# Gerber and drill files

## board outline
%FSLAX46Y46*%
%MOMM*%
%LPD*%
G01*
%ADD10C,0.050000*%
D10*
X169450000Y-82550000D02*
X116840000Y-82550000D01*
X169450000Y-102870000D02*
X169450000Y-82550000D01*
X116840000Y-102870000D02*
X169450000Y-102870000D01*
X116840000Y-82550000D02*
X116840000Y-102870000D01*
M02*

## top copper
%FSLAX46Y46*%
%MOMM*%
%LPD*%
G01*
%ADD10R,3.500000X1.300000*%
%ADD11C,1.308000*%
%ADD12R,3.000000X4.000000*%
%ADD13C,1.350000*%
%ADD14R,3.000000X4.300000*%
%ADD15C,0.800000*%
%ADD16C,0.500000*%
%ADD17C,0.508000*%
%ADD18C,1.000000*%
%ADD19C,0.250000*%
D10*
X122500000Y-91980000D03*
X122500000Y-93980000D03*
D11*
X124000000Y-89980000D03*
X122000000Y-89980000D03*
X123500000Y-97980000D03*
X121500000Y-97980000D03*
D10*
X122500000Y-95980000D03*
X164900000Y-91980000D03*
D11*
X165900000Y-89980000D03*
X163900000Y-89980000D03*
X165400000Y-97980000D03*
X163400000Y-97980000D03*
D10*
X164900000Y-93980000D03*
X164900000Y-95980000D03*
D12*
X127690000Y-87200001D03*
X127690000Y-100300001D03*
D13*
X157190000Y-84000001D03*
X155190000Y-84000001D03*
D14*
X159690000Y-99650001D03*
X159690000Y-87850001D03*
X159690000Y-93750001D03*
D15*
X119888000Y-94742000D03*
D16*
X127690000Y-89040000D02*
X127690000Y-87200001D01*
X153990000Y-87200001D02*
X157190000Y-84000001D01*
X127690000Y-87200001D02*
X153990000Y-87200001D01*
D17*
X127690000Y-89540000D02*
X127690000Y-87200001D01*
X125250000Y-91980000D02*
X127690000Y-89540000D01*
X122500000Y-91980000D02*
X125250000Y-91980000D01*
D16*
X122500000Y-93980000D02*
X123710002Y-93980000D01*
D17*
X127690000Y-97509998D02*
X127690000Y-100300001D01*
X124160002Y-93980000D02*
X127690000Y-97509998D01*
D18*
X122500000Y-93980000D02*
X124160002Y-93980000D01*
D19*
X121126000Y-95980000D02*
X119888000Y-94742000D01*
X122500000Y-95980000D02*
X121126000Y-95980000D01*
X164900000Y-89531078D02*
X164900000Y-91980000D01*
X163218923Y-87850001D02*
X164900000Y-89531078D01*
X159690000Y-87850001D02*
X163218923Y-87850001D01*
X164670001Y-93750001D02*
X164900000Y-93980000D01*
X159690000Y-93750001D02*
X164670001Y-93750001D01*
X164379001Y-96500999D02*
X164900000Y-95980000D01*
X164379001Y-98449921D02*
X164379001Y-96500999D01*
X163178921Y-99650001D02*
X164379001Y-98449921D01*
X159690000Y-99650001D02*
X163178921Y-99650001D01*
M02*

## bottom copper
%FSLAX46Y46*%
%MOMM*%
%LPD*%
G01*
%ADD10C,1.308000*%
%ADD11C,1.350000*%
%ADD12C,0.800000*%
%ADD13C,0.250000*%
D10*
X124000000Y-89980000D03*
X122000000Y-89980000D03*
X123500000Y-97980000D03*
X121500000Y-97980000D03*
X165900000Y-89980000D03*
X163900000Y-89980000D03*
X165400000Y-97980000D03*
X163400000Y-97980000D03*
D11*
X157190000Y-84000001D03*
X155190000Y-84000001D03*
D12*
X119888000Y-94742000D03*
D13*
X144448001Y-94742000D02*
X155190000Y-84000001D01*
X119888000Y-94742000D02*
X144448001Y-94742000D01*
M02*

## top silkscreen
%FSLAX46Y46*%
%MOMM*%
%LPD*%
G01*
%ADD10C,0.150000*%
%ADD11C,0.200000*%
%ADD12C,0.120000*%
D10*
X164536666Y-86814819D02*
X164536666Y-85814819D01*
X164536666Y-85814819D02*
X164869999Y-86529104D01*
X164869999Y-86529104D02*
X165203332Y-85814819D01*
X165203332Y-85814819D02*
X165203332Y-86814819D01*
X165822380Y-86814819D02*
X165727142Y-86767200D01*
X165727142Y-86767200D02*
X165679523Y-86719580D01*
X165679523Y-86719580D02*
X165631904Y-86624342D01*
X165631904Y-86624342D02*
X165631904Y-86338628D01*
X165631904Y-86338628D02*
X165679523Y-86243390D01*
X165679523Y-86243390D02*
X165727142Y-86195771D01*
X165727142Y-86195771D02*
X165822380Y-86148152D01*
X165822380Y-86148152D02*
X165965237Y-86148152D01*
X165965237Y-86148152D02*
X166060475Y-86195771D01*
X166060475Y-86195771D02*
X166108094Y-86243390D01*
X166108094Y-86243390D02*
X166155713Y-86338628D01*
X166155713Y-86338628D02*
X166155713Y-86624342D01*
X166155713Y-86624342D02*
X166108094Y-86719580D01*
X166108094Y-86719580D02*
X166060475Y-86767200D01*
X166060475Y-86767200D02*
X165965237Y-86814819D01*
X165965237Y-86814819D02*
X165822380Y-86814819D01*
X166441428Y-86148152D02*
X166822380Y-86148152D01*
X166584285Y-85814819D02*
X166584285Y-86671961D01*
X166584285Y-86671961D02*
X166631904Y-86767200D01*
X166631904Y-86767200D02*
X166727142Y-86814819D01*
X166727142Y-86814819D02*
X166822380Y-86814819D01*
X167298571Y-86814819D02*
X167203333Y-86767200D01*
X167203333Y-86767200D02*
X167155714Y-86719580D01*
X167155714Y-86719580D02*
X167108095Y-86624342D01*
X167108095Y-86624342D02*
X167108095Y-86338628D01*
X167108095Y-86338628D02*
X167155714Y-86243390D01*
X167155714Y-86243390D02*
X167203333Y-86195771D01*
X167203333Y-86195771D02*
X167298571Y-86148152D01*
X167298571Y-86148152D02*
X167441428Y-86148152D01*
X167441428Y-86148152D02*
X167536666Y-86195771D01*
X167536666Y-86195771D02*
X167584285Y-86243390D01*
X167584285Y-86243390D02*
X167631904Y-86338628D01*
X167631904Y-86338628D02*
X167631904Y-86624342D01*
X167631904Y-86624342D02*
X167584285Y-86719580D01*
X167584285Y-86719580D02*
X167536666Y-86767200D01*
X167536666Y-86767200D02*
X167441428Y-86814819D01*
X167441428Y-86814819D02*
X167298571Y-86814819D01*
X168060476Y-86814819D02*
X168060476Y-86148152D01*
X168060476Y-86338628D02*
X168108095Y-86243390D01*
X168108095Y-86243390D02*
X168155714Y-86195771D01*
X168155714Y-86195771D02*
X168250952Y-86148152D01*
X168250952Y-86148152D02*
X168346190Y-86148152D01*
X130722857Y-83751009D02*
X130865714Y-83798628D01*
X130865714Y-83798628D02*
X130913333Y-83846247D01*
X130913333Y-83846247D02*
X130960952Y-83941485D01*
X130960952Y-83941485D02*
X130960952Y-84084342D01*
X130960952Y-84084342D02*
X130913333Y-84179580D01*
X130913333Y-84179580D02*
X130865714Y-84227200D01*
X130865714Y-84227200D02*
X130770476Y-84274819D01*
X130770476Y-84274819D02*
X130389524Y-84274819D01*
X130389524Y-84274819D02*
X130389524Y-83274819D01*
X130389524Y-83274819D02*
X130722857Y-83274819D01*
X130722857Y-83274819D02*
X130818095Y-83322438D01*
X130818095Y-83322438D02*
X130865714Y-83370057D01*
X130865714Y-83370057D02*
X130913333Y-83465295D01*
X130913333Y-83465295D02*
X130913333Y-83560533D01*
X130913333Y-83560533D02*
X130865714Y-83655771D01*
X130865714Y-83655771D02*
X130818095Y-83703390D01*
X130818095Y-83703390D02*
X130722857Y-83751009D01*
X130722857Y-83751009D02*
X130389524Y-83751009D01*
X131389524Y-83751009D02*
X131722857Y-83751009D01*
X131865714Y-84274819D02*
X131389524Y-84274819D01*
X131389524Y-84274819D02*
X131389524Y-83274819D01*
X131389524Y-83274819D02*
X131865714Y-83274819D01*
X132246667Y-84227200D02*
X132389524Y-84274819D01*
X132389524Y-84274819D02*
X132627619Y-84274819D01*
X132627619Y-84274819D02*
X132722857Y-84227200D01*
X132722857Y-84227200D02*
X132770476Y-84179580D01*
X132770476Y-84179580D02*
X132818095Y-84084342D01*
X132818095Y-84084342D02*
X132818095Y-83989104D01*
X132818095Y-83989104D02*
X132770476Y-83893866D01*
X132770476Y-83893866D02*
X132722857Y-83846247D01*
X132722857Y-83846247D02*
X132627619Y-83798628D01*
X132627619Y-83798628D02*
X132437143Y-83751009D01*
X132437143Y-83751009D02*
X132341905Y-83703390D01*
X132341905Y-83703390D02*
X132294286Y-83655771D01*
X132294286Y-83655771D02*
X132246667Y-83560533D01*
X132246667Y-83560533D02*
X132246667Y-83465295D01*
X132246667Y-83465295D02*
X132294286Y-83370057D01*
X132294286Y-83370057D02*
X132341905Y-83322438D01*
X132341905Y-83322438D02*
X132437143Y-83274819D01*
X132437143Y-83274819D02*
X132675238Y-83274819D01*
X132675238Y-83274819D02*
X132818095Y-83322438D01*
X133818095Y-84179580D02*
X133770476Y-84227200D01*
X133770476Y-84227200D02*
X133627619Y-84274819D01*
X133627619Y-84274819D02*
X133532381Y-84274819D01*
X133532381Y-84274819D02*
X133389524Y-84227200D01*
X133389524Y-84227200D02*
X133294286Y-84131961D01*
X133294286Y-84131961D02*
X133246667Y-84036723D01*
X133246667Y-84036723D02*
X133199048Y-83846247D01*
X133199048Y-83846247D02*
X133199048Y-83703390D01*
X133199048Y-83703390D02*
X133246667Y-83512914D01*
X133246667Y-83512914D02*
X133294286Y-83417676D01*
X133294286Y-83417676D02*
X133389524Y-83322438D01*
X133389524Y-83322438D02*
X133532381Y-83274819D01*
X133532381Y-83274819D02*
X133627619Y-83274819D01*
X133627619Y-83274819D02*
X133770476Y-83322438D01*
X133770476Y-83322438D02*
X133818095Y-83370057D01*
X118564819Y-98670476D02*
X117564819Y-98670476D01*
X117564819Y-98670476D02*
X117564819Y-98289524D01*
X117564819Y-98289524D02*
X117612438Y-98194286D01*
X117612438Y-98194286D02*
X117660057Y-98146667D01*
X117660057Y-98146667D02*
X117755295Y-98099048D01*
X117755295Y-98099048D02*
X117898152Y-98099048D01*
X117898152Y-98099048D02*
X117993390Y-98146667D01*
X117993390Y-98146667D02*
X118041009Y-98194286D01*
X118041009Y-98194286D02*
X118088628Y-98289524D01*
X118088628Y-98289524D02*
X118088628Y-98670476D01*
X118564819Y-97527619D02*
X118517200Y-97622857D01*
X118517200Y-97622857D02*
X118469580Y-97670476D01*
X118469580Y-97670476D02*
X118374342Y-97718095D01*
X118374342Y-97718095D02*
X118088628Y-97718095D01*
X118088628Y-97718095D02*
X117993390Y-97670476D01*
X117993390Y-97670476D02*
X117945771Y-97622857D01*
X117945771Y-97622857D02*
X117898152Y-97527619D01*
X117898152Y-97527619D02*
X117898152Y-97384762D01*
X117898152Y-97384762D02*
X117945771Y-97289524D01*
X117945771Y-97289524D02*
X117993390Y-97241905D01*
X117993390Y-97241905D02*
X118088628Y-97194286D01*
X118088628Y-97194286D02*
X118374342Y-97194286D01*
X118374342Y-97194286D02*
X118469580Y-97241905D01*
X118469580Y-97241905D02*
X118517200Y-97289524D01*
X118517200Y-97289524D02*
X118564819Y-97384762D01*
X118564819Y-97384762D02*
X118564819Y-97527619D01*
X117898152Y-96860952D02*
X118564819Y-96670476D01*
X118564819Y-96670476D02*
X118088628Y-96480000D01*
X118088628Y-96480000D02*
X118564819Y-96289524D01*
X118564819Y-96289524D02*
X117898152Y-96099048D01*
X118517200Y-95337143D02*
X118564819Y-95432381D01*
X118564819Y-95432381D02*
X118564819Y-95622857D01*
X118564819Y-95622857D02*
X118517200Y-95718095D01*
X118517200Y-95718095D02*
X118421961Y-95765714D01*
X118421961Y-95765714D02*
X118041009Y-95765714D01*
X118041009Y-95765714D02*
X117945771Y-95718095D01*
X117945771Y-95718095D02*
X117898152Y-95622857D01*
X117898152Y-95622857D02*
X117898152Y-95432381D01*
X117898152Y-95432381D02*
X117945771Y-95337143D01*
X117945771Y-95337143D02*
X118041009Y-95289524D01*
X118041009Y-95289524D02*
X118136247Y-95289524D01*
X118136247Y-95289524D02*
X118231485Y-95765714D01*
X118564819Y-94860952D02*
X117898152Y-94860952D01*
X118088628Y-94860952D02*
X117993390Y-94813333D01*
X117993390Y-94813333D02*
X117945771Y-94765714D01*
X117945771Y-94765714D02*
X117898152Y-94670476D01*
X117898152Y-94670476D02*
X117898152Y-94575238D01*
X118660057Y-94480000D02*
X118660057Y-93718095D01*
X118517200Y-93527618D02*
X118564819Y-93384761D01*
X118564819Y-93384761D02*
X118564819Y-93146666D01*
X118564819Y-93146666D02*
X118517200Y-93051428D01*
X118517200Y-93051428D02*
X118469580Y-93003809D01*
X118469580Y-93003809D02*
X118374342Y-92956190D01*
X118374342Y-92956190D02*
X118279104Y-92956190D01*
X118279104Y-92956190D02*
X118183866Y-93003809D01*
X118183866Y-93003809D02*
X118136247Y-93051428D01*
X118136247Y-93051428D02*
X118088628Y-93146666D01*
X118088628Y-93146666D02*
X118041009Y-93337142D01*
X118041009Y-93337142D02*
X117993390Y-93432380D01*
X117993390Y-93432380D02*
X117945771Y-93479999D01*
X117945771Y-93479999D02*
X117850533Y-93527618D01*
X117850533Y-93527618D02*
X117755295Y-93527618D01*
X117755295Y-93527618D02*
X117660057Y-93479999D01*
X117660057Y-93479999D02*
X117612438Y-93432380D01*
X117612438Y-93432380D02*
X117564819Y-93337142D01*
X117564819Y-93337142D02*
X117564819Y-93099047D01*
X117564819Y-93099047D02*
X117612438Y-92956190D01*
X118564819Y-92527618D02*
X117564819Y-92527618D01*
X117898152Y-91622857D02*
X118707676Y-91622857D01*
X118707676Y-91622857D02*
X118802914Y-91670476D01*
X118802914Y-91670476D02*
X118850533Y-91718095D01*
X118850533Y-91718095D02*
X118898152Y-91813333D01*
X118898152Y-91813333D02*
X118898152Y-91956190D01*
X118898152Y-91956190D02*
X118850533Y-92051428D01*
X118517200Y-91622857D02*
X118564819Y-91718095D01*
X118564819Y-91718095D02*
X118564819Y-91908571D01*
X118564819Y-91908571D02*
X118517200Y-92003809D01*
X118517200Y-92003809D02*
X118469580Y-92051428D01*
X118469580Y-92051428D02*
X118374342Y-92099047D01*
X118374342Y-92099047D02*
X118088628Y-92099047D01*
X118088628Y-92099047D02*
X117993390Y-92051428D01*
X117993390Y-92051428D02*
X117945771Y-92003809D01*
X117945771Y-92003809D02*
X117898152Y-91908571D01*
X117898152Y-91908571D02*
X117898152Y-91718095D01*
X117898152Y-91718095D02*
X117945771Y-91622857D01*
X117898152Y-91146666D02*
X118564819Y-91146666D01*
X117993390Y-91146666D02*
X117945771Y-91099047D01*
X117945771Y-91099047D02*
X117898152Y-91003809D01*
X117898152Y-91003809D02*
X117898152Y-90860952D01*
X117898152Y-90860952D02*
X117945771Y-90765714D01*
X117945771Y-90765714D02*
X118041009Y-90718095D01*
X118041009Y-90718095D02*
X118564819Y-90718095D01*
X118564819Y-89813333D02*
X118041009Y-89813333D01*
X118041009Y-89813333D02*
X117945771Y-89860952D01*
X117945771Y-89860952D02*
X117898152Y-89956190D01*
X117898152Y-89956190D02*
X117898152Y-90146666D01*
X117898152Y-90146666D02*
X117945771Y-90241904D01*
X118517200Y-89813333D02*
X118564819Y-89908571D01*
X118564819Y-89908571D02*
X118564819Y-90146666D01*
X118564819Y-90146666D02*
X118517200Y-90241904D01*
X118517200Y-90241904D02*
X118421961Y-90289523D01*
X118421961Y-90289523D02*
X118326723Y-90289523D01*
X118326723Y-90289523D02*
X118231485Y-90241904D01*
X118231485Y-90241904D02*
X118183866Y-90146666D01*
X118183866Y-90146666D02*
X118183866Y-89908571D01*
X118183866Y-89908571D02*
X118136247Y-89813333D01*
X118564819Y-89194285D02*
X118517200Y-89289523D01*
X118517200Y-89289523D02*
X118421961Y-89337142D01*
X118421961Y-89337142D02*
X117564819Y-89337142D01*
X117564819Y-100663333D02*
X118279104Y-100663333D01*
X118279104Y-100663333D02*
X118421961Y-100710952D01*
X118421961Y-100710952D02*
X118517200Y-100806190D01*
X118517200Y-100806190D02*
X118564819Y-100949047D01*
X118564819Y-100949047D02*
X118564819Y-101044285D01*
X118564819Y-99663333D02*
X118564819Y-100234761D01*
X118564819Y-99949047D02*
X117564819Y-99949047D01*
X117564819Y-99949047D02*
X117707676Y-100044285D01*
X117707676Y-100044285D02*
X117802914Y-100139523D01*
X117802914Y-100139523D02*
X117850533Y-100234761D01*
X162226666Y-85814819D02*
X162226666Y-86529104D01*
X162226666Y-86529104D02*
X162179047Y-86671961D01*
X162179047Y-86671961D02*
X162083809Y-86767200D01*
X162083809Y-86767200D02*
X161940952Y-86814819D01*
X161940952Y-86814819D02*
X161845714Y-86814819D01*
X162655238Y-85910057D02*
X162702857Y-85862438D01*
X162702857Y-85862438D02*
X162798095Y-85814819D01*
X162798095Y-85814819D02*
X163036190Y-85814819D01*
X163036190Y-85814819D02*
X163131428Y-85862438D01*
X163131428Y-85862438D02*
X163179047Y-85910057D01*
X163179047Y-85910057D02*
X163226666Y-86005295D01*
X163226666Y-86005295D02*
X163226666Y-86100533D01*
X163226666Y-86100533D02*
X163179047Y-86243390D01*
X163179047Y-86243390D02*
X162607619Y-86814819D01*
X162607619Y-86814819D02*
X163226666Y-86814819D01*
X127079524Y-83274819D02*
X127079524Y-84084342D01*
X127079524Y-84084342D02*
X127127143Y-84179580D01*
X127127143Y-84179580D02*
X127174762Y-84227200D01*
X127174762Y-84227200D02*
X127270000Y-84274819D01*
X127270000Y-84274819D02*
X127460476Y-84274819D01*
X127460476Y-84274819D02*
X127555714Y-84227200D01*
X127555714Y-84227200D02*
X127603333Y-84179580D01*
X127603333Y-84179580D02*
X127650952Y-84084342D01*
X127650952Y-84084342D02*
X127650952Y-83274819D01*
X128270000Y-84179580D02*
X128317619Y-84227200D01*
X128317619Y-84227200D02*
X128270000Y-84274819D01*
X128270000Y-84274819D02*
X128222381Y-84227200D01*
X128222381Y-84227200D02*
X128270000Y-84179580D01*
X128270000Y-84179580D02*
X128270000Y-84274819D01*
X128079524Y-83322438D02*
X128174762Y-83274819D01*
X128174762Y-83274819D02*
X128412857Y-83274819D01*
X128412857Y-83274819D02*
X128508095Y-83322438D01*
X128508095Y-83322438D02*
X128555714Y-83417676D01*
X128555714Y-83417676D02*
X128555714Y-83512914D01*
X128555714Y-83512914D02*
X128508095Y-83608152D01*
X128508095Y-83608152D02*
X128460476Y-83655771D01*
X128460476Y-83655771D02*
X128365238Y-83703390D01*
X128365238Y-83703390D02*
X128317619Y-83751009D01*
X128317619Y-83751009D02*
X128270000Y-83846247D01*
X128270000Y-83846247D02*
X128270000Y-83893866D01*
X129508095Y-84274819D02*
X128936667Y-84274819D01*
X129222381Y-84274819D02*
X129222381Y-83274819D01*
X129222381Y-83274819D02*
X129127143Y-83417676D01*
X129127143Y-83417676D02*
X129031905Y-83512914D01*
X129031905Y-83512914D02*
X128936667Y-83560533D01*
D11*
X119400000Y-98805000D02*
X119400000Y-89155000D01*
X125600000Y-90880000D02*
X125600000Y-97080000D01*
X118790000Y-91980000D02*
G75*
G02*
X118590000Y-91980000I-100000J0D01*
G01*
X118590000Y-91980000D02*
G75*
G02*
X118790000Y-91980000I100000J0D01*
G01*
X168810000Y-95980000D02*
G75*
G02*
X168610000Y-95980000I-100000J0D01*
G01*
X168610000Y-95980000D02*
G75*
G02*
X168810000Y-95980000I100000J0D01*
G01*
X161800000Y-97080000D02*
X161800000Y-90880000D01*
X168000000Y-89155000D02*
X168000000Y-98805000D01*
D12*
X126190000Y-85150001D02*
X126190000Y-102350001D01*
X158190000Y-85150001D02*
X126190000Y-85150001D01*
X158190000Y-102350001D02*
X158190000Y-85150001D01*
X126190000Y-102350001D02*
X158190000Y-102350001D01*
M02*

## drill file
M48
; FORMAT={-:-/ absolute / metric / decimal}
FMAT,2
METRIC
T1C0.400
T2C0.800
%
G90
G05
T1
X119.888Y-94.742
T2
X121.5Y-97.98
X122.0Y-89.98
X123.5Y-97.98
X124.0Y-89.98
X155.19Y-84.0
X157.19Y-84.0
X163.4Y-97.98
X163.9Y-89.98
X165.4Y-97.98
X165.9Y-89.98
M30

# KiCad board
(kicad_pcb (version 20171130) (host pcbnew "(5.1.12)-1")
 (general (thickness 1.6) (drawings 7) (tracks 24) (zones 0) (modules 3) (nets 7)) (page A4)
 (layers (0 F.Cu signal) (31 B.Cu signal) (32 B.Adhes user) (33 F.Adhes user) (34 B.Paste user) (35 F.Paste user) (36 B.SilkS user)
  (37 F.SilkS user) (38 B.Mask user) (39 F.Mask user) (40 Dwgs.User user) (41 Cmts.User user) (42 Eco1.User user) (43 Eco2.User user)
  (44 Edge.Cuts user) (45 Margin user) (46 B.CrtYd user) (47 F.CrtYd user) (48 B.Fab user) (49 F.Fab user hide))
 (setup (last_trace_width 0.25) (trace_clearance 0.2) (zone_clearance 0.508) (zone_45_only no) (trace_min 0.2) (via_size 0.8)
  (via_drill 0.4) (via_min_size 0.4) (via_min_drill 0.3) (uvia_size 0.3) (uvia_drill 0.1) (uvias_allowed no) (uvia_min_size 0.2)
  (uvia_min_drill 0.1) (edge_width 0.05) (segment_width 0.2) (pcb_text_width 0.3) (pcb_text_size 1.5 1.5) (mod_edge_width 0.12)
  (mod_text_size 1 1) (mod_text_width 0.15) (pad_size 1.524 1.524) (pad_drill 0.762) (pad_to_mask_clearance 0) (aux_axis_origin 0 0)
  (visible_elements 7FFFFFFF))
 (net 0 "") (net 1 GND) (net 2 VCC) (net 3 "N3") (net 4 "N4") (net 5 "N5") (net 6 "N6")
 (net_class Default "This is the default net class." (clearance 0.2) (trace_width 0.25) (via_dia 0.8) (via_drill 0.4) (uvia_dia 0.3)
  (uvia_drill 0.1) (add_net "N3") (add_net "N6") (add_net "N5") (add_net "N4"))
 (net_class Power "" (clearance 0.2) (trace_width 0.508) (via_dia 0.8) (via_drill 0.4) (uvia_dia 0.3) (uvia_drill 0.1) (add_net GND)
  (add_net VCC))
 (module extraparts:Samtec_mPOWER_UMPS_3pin (layer F.Cu) (at 122.5 93.98 270)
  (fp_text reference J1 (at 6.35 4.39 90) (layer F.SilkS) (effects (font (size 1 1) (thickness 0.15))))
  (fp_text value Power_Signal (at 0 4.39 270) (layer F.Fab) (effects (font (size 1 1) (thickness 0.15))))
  (fp_line (start 4.825 3.1) (end -4.825 3.1) (layer F.SilkS) (width 0.2))
  (fp_line (start -3.1 -3.1) (end 3.1 -3.1) (layer F.SilkS) (width 0.2))
  (fp_circle (center -2 3.81) (end -1.9 3.81) (layer F.SilkS) (width 0.2))
  (pad 1 smd rect (at -2 0 270) (size 1.3 3.5) (layers F.Cu F.Paste F.Mask) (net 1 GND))
  (pad 2 smd rect (at 0 0 270) (size 1.3 3.5) (layers F.Cu F.Paste F.Mask) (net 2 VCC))
  (pad "" thru_hole circle (at -4 -1.5 270) (size 1.308 1.308) (drill 0.8) (layers *.Cu *.Mask))
  (pad "" thru_hole circle (at -4 0.5 270) (size 1.308 1.308) (drill 0.8) (layers *.Cu *.Mask))
  (pad "" thru_hole circle (at 4 -1 270) (size 1.308 1.308) (drill 0.8) (layers *.Cu *.Mask))
  (pad "" thru_hole circle (at 4 1 270) (size 1.308 1.308) (drill 0.8) (layers *.Cu *.Mask))
  (pad 3 smd rect (at 2 0 270) (size 1.3 3.5) (layers F.Cu F.Paste F.Mask) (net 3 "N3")))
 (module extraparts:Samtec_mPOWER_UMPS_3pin (layer F.Cu) (at 164.9 93.98 90)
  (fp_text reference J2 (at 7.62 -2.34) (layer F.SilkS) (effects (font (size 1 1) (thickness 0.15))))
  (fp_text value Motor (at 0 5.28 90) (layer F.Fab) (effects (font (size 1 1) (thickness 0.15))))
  (fp_circle (center -2 3.81) (end -1.9 3.81) (layer F.SilkS) (width 0.2))
  (fp_line (start -3.1 -3.1) (end 3.1 -3.1) (layer F.SilkS) (width 0.2))
  (fp_line (start 4.825 3.1) (end -4.825 3.1) (layer F.SilkS) (width 0.2))
  (pad 3 smd rect (at 2 0 90) (size 1.3 3.5) (layers F.Cu F.Paste F.Mask) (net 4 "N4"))
  (pad "" thru_hole circle (at 4 1 90) (size 1.308 1.308) (drill 0.8) (layers *.Cu *.Mask))
  (pad "" thru_hole circle (at 4 -1 90) (size 1.308 1.308) (drill 0.8) (layers *.Cu *.Mask))
  (pad "" thru_hole circle (at -4 0.5 90) (size 1.308 1.308) (drill 0.8) (layers *.Cu *.Mask))
  (pad "" thru_hole circle (at -4 -1.5 90) (size 1.308 1.308) (drill 0.8) (layers *.Cu *.Mask))
  (pad 2 smd rect (at 0 0 90) (size 1.3 3.5) (layers F.Cu F.Paste F.Mask) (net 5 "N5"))
  (pad 1 smd rect (at -2 0 90) (size 1.3 3.5) (layers F.Cu F.Paste F.Mask) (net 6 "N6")))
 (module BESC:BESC (layer F.Cu) (at 142.19 93.750001 180)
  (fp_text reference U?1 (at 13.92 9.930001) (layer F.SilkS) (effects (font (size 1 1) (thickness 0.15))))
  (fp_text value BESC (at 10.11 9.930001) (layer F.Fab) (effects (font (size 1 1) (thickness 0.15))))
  (fp_line (start 16 8.6) (end 16 -8.6) (layer F.SilkS) (width 0.12))
  (fp_line (start -16 8.6) (end 16 8.6) (layer F.SilkS) (width 0.12))
  (fp_line (start -16 -8.6) (end -16 8.6) (layer F.SilkS) (width 0.12))
  (fp_line (start 16 -8.6) (end -16 -8.6) (layer F.SilkS) (width 0.12))
  (pad 1 smd rect (at 14.5 6.55 180) (size 3 4) (layers F.Cu F.Paste F.Mask) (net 1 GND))
  (pad 4 smd rect (at 14.5 -6.55 180) (size 3 4) (layers F.Cu F.Paste F.Mask) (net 2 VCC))
  (pad 3 thru_hole circle (at -15 9.75) (size 1.35 1.35) (drill 0.8) (layers *.Cu *.Mask) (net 1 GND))
  (pad 2 thru_hole circle (at -13 9.75) (size 1.35 1.35) (drill 0.8) (layers *.Cu *.Mask) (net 3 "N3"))
  (pad 5 smd rect (at -17.5 -5.9 180) (size 3 4.3) (layers F.Cu F.Paste F.Mask) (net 6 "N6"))
  (pad 7 smd rect (at -17.5 5.9 180) (size 3 4.3) (layers F.Cu F.Paste F.Mask) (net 4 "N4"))
  (pad 6 smd rect (at -17.5 0 180) (size 3 4.3) (layers F.Cu F.Paste F.Mask) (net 5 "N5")))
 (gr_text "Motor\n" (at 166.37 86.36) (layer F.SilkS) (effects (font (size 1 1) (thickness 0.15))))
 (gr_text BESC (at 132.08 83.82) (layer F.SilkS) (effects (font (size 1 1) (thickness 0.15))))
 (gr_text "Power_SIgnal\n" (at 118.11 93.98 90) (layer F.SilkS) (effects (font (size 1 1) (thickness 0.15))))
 (gr_line (start 169.45 82.55) (end 116.84 82.55) (layer Edge.Cuts) (width 0.05))
 (gr_line (start 169.45 102.87) (end 169.45 82.55) (layer Edge.Cuts) (width 0.05))
 (gr_line (start 116.84 102.87) (end 169.45 102.87) (layer Edge.Cuts) (width 0.05))
 (gr_line (start 116.84 82.55) (end 116.84 102.87) (layer Edge.Cuts) (width 0.05))
 (segment (start 127.69 89.04) (end 127.69 87.200001) (width 0.5) (layer F.Cu) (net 1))
 (segment (start 153.99 87.200001) (end 157.19 84.000001) (width 0.5) (layer F.Cu) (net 1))
 (segment (start 127.69 87.200001) (end 153.99 87.200001) (width 0.5) (layer F.Cu) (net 1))
 (segment (start 127.69 89.54) (end 127.69 87.200001) (width 0.508) (layer F.Cu) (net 1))
 (segment (start 125.25 91.98) (end 127.69 89.54) (width 0.508) (layer F.Cu) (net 1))
 (segment (start 122.5 91.98) (end 125.25 91.98) (width 0.508) (layer F.Cu) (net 1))
 (segment (start 122.5 93.98) (end 123.710002 93.98) (width 0.5) (layer F.Cu) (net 2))
 (segment (start 127.69 97.509998) (end 127.69 100.300001) (width 0.508) (layer F.Cu) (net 2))
 (segment (start 124.160002 93.98) (end 127.69 97.509998) (width 0.508) (layer F.Cu) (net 2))
 (segment (start 122.5 93.98) (end 124.160002 93.98) (width 1) (layer F.Cu) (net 2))
 (via (at 119.888 94.742) (size 0.8) (drill 0.4) (layers F.Cu B.Cu) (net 3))
 (segment (start 121.126 95.98) (end 119.888 94.742) (width 0.25) (layer F.Cu) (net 3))
 (segment (start 122.5 95.98) (end 121.126 95.98) (width 0.25) (layer F.Cu) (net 3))
 (segment (start 144.448001 94.742) (end 155.19 84.000001) (width 0.25) (layer B.Cu) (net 3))
 (segment (start 119.888 94.742) (end 144.448001 94.742) (width 0.25) (layer B.Cu) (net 3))
 (segment (start 164.9 89.531078) (end 164.9 91.98) (width 0.25) (layer F.Cu) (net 4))
 (segment (start 163.218923 87.850001) (end 164.9 89.531078) (width 0.25) (layer F.Cu) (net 4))
 (segment (start 159.69 87.850001) (end 163.218923 87.850001) (width 0.25) (layer F.Cu) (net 4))
 (segment (start 164.670001 93.750001) (end 164.9 93.98) (width 0.25) (layer F.Cu) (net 5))
 (segment (start 159.69 93.750001) (end 164.670001 93.750001) (width 0.25) (layer F.Cu) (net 5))
 (segment (start 164.379001 96.500999) (end 164.9 95.98) (width 0.25) (layer F.Cu) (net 6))
 (segment (start 164.379001 98.449921) (end 164.379001 96.500999) (width 0.25) (layer F.Cu) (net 6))
 (segment (start 163.178921 99.650001) (end 164.379001 98.449921) (width 0.25) (layer F.Cu) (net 6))
 (segment (start 159.69 99.650001) (end 163.178921 99.650001) (width 0.25) (layer F.Cu) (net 6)))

